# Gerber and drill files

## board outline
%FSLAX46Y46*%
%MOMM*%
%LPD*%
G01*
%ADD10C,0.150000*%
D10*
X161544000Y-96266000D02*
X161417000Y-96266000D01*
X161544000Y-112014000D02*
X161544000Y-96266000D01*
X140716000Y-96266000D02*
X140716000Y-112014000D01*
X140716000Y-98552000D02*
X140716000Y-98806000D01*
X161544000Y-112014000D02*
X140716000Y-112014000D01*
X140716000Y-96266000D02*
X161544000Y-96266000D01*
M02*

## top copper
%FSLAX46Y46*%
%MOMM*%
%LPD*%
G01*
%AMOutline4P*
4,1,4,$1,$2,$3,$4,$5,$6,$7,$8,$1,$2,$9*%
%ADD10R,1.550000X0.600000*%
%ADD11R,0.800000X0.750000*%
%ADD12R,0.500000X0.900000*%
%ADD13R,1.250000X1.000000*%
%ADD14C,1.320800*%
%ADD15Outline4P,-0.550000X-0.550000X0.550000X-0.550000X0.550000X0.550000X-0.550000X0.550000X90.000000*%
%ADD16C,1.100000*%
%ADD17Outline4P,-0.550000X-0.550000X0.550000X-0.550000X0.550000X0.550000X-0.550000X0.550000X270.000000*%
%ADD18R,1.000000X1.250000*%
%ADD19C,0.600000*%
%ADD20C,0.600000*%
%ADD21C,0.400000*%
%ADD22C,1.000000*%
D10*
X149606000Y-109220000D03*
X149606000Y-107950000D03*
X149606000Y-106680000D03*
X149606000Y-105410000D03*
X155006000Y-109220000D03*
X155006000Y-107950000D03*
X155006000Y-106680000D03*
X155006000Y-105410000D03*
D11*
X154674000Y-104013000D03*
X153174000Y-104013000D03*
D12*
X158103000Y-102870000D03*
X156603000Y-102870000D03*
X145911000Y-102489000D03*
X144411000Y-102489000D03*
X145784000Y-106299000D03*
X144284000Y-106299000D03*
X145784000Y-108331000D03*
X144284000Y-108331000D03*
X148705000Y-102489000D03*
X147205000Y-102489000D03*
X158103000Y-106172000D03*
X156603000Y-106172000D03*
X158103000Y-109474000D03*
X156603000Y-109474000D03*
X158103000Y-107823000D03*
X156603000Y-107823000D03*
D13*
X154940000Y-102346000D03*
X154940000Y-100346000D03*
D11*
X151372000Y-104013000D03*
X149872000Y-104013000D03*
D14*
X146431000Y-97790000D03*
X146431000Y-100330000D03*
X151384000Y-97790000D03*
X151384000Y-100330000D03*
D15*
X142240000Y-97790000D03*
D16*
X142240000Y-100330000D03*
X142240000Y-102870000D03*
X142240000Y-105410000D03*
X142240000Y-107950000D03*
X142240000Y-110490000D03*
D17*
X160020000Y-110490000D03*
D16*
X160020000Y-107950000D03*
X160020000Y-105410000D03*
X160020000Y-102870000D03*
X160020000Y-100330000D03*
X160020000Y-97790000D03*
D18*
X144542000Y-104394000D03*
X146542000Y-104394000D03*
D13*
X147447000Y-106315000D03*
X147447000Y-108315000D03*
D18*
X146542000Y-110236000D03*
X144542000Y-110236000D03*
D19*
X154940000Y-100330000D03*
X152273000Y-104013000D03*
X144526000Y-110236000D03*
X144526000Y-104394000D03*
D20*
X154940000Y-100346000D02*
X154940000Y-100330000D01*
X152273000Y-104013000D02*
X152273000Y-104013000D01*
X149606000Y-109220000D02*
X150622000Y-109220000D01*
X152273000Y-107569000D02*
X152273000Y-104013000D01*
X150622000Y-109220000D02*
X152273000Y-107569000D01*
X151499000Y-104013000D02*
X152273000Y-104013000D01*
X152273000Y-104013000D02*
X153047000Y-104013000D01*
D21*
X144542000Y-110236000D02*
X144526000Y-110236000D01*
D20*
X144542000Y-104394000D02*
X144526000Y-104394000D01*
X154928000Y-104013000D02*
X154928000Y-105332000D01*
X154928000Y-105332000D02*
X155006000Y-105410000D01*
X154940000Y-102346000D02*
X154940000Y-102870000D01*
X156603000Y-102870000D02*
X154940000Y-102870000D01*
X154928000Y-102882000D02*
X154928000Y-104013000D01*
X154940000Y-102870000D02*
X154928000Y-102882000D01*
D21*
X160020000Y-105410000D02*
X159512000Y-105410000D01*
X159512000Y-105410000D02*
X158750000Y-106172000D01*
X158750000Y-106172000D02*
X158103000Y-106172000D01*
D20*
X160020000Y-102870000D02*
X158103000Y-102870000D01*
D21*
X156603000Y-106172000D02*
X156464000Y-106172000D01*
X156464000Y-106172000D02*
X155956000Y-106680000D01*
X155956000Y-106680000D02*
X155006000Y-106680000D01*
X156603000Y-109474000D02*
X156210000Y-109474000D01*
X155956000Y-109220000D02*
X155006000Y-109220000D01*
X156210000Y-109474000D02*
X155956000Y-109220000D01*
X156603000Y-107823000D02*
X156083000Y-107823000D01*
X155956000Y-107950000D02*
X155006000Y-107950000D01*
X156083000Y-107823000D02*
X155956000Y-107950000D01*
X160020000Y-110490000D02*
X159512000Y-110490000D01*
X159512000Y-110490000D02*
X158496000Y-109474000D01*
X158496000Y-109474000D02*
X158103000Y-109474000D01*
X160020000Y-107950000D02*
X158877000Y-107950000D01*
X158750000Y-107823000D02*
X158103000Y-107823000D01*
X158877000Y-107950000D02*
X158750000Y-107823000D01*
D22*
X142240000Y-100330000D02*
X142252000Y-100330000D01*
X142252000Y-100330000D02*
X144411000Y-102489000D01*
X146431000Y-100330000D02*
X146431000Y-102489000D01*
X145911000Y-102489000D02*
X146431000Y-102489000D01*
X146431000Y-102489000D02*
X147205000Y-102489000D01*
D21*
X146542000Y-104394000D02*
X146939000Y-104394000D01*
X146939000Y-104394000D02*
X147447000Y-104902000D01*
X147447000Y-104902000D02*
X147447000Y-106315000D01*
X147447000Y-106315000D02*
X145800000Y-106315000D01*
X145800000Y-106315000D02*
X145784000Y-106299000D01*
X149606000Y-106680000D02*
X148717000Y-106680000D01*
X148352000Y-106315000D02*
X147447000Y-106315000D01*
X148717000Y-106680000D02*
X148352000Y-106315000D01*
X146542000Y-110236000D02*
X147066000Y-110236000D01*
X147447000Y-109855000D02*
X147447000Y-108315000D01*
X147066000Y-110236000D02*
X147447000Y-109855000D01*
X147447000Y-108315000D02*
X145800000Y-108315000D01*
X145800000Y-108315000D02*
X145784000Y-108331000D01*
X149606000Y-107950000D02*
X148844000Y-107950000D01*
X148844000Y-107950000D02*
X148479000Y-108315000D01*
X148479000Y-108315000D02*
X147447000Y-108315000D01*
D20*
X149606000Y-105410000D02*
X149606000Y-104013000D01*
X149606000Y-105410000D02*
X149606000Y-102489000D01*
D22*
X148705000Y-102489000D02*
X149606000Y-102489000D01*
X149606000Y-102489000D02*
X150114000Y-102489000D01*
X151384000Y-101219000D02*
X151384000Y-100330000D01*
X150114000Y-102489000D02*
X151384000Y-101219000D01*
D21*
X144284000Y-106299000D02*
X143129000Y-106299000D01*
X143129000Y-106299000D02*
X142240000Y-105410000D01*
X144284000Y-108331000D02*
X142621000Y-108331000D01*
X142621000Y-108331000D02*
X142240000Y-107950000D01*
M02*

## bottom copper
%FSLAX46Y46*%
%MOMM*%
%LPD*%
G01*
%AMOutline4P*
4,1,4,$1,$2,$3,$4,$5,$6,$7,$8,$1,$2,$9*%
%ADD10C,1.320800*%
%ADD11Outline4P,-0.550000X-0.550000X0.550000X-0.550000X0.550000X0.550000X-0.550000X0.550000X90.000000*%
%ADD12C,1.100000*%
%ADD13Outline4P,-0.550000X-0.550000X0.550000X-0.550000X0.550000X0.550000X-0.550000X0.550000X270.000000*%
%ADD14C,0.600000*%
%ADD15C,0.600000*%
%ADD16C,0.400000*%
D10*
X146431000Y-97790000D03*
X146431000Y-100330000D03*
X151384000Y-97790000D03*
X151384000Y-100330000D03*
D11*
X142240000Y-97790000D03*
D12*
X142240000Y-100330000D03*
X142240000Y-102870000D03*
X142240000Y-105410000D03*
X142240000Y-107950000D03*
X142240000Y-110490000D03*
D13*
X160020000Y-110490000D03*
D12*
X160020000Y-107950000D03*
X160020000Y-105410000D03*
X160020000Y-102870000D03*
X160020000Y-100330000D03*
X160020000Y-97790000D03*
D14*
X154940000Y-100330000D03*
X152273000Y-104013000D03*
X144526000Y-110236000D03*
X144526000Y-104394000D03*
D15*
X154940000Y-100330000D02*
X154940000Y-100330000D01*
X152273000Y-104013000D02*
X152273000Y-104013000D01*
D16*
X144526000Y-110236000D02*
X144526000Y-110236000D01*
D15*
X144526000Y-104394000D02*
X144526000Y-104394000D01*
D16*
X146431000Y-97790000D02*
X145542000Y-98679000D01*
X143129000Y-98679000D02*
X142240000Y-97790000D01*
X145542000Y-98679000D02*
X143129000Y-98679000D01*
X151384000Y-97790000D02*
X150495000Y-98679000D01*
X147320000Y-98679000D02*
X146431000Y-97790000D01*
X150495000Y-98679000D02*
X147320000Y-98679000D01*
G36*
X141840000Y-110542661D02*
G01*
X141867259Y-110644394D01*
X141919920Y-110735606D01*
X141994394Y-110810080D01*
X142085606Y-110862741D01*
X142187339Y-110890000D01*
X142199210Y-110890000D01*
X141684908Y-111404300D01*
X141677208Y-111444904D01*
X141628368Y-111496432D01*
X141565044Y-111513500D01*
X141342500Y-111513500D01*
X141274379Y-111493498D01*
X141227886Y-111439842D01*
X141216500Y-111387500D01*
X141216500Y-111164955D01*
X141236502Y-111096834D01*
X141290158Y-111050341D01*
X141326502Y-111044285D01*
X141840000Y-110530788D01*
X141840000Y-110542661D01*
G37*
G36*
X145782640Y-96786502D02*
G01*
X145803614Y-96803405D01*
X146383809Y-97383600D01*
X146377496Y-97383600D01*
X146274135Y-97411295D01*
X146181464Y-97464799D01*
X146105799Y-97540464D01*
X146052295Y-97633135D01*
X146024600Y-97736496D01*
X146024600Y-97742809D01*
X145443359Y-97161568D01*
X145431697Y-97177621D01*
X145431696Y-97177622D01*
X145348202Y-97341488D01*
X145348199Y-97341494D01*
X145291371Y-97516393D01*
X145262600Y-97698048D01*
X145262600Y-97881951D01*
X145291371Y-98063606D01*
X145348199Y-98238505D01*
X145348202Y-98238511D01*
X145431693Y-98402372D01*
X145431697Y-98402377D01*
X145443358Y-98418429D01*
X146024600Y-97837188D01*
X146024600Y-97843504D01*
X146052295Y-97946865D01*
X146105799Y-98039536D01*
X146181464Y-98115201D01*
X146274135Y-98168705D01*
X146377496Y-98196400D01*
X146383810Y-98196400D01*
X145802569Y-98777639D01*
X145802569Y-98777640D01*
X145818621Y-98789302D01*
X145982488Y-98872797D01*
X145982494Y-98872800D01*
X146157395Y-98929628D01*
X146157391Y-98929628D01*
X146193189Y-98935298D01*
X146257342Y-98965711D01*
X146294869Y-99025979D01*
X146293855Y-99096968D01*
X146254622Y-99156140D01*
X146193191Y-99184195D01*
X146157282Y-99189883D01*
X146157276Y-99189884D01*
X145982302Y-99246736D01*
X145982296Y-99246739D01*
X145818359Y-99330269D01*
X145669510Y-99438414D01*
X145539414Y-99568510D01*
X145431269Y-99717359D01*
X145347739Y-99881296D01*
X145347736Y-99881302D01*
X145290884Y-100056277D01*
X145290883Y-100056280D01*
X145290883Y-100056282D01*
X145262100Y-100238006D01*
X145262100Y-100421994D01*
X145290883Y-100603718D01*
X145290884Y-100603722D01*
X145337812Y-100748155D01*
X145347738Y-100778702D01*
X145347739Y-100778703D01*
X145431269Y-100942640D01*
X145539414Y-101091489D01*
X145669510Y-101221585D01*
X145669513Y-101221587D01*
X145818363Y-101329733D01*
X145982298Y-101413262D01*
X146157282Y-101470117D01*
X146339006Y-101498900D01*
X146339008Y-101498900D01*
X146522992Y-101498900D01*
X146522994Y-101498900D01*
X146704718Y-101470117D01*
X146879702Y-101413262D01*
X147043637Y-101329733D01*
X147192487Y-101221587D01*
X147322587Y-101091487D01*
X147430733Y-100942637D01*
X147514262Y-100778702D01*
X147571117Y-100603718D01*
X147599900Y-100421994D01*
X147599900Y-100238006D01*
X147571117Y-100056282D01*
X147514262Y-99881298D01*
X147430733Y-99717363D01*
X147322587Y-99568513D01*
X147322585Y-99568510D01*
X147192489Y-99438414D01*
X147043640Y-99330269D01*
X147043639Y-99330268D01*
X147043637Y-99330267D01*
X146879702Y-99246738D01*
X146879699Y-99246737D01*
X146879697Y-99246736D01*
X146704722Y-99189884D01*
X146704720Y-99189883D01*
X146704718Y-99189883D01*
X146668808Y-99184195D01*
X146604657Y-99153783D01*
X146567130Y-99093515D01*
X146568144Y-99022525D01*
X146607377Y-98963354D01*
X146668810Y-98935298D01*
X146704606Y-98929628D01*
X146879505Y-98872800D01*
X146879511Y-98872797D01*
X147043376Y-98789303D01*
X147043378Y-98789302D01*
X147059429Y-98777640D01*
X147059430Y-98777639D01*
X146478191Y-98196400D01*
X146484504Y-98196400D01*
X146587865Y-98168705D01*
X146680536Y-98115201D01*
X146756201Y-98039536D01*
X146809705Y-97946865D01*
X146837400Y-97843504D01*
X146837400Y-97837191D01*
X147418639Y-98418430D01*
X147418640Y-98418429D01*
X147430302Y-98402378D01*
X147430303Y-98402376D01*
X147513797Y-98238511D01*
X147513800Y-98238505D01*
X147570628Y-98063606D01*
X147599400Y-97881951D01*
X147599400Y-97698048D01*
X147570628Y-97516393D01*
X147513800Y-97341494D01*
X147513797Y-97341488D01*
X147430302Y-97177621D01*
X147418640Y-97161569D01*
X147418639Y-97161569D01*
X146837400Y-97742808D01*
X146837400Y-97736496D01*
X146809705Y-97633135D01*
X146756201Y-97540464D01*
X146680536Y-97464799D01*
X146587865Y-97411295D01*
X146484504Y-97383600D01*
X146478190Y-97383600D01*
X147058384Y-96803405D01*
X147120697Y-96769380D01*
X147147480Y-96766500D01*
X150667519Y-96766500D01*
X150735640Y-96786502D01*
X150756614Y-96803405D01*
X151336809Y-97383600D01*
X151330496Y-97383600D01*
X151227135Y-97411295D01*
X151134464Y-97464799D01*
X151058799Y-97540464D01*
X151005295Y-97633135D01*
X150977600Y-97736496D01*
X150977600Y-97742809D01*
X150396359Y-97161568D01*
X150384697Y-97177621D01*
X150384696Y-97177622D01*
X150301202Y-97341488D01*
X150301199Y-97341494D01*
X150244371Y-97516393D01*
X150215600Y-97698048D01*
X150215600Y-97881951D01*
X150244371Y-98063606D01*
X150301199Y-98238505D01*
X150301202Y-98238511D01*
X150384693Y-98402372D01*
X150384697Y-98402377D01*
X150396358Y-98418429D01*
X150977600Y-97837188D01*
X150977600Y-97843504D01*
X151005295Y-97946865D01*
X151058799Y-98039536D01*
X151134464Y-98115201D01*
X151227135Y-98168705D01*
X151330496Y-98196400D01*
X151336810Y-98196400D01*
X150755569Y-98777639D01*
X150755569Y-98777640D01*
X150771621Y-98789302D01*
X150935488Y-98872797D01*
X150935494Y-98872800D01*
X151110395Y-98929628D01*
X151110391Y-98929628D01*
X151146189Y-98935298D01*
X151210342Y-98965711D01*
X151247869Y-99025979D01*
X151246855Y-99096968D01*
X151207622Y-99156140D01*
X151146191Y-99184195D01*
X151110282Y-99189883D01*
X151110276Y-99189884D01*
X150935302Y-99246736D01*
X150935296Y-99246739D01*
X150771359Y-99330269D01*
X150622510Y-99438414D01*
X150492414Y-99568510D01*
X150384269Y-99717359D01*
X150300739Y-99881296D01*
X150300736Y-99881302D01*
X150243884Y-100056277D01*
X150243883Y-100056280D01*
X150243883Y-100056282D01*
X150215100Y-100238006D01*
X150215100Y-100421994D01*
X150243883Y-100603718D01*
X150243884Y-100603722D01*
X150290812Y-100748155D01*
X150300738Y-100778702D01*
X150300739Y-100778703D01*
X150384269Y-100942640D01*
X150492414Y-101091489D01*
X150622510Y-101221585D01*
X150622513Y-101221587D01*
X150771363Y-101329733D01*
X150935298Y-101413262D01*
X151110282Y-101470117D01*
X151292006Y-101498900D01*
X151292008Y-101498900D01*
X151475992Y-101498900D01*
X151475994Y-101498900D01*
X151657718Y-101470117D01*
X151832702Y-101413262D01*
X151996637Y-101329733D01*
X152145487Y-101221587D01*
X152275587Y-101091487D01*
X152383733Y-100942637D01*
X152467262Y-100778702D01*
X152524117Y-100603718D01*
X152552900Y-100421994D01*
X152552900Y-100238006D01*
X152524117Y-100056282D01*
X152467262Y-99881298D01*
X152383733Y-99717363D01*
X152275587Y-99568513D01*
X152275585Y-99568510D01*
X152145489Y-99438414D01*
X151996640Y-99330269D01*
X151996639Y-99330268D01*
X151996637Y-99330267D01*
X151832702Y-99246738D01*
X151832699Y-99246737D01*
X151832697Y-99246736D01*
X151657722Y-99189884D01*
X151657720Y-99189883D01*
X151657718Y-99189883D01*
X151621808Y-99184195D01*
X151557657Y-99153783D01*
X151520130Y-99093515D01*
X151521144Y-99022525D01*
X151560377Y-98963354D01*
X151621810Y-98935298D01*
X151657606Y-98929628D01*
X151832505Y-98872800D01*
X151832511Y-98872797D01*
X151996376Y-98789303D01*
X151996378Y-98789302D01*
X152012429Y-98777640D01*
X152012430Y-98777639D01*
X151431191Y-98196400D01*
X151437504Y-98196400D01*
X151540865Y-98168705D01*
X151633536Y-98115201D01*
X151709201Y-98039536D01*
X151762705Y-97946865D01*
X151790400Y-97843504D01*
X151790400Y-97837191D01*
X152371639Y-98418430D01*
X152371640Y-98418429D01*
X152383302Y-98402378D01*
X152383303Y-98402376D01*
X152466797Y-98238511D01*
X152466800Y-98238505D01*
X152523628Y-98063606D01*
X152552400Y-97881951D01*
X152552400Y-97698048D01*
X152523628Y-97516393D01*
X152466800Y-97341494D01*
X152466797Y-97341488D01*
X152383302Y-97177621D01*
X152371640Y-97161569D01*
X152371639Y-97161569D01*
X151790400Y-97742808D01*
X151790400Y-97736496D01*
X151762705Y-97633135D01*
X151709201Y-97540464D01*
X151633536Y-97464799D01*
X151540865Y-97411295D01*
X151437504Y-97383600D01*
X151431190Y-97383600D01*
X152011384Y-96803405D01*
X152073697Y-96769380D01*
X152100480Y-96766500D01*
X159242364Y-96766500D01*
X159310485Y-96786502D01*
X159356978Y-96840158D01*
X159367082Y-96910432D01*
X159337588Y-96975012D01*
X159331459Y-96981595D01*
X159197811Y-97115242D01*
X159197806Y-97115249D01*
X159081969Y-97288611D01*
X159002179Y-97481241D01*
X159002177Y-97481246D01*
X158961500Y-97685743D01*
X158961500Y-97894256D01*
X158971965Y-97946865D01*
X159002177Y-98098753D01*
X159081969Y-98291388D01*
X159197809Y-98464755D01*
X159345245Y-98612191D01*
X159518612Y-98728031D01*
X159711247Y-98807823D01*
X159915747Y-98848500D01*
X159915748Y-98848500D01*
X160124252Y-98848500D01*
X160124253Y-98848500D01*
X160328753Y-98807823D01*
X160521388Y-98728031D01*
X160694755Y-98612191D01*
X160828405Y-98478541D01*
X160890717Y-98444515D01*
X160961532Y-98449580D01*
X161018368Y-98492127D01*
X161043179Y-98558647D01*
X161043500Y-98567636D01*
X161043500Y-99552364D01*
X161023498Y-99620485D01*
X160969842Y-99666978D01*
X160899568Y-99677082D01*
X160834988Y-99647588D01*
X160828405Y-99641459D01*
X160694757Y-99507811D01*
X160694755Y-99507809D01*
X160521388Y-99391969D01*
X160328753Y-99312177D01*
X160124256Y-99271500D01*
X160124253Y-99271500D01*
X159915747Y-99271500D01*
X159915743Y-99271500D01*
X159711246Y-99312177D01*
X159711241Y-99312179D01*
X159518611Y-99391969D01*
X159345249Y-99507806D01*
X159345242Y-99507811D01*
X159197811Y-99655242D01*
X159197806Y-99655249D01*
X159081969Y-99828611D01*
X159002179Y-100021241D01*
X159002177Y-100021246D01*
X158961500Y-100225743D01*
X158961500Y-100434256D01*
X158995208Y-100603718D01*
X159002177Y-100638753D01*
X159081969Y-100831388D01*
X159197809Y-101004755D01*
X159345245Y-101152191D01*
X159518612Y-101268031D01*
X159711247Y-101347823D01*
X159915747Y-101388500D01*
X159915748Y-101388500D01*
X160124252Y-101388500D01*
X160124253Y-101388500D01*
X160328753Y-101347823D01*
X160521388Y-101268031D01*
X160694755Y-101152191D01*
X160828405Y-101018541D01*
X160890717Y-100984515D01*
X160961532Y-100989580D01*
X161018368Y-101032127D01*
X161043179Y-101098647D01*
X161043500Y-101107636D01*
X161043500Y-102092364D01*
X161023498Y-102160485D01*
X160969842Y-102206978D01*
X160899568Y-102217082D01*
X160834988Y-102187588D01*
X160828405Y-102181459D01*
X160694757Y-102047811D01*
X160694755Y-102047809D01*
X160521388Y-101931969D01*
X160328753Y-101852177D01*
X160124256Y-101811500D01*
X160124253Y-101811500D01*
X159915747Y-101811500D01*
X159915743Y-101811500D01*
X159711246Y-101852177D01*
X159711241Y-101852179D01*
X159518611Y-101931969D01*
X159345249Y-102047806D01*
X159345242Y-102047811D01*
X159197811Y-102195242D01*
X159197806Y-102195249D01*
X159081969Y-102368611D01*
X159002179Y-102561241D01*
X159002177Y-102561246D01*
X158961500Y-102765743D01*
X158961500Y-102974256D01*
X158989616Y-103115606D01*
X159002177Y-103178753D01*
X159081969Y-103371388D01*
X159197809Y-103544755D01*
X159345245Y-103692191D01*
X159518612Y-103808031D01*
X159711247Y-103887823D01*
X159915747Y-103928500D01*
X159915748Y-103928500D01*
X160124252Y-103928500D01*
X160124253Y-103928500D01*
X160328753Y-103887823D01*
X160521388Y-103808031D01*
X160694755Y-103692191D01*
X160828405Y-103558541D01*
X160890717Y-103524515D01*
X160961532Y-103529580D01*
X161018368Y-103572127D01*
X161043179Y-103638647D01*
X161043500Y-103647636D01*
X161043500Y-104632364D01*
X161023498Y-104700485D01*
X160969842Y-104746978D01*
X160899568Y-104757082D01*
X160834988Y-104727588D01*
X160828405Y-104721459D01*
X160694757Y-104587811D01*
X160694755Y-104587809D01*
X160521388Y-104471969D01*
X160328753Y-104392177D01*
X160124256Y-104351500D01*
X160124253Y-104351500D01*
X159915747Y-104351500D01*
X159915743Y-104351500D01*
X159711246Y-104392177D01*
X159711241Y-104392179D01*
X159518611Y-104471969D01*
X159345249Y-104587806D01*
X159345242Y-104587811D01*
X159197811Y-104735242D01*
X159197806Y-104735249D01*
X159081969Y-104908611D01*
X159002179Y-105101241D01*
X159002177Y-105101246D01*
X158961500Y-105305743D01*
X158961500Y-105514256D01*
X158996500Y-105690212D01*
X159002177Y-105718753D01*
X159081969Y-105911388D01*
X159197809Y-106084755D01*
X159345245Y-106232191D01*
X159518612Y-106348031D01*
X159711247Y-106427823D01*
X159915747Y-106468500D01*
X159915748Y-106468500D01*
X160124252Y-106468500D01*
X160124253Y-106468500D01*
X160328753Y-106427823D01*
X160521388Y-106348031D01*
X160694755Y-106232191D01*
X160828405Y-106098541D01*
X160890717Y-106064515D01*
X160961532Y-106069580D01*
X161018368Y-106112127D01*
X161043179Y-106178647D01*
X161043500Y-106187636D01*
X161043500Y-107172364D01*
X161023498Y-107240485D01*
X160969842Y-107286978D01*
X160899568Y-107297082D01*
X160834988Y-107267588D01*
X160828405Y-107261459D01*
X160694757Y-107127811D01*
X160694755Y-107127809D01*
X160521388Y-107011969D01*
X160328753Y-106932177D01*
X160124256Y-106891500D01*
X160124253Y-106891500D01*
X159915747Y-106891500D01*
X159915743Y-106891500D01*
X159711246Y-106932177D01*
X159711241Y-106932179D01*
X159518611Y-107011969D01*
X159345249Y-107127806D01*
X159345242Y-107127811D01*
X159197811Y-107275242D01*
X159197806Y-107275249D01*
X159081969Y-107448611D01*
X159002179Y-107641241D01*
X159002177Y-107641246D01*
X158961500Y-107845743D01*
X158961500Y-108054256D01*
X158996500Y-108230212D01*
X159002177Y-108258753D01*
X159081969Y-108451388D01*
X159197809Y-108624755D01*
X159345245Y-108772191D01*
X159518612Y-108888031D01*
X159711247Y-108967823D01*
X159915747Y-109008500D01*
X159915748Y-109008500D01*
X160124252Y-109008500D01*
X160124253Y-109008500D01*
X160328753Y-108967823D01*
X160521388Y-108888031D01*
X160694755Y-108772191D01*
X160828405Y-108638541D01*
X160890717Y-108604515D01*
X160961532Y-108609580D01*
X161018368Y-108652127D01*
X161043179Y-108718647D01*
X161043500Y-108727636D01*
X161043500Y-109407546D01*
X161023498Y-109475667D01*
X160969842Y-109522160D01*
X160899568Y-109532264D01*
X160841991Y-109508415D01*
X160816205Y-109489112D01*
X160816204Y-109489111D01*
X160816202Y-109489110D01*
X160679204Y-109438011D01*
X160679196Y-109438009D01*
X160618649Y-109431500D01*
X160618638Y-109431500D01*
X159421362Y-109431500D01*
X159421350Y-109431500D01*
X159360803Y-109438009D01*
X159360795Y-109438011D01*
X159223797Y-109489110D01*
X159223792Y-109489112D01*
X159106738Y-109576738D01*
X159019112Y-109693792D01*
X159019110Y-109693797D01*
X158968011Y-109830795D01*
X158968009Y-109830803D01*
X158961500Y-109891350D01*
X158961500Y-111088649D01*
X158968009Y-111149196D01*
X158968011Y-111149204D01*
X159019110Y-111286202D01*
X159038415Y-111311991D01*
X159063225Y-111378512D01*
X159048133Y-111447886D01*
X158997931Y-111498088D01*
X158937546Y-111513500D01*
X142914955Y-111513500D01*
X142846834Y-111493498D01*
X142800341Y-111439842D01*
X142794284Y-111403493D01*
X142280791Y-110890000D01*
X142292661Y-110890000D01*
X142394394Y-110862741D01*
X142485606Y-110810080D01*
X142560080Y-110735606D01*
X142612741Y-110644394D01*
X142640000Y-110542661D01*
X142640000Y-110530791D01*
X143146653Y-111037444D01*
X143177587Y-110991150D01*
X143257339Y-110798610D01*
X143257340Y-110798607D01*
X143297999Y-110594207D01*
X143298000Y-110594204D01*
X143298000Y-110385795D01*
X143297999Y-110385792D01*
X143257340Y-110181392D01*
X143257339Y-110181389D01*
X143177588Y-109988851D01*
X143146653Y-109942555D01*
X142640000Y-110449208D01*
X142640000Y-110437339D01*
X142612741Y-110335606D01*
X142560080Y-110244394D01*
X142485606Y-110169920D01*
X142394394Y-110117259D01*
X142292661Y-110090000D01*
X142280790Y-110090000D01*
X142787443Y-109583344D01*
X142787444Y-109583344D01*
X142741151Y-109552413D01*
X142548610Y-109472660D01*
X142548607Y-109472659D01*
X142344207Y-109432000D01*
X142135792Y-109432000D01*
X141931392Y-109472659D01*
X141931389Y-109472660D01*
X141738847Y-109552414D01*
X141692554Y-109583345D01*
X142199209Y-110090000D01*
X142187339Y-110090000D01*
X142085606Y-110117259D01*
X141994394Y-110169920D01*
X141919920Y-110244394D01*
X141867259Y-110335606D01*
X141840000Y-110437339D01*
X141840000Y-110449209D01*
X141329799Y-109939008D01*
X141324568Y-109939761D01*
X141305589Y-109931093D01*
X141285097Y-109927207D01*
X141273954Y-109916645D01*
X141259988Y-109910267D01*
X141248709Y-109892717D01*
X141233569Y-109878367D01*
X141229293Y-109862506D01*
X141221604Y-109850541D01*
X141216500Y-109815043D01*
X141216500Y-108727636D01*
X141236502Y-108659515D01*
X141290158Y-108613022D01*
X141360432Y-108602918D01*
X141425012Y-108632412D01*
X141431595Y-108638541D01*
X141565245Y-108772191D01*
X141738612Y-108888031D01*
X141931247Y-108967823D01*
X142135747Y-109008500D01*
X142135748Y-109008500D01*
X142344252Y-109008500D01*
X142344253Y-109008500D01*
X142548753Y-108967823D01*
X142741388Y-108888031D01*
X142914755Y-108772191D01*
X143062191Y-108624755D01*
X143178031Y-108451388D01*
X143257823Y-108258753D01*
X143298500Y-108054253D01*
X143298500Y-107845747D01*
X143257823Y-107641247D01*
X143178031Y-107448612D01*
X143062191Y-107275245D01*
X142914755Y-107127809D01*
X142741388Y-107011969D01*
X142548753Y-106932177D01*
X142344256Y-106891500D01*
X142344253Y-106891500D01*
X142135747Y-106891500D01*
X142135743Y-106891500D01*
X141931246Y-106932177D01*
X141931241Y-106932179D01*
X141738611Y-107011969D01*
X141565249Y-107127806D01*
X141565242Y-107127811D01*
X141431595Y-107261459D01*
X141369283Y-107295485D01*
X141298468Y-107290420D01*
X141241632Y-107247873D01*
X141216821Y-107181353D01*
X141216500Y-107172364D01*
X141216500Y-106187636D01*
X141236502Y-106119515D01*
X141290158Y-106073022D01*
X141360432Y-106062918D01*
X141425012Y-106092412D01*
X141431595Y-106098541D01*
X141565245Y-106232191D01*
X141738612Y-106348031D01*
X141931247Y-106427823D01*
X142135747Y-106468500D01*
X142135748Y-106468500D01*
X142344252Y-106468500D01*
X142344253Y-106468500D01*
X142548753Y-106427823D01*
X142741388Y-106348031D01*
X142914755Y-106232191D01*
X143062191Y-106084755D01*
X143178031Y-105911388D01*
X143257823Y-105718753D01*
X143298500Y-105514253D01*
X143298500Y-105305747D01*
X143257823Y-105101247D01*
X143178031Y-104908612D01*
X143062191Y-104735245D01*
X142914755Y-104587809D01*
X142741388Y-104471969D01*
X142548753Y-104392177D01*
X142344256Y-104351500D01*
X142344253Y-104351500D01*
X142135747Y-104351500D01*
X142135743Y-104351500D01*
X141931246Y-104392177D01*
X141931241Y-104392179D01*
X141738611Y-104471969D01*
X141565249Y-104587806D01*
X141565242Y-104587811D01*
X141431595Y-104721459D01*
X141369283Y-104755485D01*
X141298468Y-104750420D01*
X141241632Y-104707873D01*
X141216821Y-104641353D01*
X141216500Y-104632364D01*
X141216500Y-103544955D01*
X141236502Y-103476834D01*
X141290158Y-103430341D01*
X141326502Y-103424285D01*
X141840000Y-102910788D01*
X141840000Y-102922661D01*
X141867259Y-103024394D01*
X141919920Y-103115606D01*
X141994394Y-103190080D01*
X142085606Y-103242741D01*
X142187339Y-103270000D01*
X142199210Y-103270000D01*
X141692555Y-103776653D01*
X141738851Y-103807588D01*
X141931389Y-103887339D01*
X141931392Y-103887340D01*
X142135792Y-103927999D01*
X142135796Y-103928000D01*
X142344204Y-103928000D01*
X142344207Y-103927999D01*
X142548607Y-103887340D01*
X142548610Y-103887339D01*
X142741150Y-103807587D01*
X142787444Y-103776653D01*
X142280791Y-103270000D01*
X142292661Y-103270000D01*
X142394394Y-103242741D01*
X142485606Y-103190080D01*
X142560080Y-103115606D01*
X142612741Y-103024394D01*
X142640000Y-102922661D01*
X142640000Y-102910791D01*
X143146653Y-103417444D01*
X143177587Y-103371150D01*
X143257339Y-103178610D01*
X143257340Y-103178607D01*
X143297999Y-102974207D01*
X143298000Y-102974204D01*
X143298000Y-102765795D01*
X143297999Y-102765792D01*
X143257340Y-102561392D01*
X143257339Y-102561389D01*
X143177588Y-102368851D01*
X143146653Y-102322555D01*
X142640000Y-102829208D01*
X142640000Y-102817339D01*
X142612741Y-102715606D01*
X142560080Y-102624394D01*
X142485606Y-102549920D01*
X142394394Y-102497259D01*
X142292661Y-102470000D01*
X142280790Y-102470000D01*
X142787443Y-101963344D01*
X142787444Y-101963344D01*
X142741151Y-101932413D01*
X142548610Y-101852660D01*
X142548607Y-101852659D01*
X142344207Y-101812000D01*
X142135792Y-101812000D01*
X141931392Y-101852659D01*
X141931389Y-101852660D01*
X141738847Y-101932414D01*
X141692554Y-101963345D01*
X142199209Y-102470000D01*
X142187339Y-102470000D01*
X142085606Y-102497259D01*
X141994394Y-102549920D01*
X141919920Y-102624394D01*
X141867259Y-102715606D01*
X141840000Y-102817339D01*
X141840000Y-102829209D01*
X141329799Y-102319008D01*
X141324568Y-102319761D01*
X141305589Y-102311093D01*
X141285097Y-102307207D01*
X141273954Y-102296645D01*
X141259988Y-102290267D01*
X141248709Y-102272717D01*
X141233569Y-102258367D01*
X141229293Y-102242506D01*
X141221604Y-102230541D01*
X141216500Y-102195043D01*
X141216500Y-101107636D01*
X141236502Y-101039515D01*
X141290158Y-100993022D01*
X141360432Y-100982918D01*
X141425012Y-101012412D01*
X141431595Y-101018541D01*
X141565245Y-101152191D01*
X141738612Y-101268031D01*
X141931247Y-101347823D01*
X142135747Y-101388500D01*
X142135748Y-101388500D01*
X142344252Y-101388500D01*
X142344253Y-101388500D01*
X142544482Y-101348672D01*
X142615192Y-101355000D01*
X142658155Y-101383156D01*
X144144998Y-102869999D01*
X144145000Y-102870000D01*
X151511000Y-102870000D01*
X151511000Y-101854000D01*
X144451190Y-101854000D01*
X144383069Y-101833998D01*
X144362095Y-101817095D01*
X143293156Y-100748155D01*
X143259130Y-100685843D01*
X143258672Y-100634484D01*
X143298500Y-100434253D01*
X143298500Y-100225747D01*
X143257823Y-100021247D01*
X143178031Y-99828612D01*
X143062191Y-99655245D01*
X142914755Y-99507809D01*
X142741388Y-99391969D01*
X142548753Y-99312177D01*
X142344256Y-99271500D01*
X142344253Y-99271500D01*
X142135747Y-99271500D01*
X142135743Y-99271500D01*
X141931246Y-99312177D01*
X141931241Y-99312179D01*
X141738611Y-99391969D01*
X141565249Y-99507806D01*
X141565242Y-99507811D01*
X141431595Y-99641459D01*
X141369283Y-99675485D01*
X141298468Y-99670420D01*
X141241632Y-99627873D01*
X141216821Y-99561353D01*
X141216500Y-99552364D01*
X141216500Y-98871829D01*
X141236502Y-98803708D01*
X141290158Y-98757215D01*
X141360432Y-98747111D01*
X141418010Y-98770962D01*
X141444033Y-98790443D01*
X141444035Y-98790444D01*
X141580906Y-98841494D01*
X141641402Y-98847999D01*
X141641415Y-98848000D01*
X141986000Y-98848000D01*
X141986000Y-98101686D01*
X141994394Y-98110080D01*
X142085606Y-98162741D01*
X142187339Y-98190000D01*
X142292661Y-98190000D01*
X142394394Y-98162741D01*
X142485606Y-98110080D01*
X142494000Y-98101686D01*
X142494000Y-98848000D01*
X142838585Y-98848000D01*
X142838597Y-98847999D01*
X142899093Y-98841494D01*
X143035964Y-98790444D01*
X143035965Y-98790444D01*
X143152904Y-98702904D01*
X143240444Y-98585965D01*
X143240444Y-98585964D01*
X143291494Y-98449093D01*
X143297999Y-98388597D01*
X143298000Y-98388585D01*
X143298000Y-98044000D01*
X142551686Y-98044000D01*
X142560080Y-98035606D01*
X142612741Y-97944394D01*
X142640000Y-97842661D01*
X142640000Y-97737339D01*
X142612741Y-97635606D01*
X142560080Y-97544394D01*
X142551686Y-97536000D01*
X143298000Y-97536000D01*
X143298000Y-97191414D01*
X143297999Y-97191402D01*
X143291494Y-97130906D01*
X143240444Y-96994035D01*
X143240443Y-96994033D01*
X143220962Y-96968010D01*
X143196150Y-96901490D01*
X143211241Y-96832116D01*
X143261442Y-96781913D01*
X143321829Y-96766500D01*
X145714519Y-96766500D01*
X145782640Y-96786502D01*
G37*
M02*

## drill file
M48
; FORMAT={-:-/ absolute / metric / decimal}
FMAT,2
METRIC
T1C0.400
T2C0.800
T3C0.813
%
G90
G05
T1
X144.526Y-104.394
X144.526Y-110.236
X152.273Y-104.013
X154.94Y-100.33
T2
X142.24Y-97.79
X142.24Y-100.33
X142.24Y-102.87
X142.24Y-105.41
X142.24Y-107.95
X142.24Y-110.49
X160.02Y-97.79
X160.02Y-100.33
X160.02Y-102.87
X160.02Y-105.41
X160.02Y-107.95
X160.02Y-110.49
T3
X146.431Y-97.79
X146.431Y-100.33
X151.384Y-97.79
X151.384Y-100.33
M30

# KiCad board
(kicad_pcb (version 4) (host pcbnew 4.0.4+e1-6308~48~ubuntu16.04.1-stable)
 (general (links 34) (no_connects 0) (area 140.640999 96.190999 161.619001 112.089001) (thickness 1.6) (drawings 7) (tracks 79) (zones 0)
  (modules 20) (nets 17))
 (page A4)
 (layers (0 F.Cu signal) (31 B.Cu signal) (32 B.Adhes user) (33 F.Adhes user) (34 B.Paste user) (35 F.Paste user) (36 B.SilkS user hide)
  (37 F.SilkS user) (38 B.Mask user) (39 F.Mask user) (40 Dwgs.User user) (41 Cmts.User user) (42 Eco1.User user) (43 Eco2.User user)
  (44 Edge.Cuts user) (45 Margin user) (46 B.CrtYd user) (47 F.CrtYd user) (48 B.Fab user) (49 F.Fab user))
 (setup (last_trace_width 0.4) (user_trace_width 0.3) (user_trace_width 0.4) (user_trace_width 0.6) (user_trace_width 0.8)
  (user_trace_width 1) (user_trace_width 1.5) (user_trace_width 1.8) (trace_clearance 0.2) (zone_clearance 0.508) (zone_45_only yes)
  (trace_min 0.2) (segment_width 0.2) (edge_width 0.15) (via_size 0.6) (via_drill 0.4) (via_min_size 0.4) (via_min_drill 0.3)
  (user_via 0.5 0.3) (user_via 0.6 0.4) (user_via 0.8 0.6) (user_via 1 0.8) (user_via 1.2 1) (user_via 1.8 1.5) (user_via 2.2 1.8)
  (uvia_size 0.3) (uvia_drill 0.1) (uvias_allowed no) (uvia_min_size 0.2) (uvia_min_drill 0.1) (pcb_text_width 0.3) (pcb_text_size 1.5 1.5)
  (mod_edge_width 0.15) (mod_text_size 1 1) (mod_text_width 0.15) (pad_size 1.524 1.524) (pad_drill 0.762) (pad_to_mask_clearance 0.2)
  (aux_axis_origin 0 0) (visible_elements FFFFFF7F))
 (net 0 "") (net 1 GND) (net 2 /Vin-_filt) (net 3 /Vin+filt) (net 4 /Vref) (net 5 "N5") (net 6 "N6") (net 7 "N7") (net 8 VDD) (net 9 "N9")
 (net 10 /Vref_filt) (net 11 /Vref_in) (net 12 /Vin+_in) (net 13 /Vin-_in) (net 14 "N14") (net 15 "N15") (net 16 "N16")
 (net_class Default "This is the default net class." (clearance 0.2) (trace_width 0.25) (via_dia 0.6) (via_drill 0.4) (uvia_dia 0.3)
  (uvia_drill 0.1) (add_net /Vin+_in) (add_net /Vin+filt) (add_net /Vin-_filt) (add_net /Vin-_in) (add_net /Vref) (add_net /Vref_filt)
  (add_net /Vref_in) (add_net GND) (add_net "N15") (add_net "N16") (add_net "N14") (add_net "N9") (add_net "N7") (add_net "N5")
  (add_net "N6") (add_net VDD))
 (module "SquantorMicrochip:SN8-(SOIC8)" (layer F.Cu) (at 152.273 107.315)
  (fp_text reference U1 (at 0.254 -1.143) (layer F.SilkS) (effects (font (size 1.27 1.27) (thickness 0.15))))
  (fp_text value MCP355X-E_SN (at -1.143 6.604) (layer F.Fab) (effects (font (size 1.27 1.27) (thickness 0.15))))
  (pad 4 smd rect (at -2.667 1.905 270) (size 0.6 1.55) (layers F.Cu F.Paste F.Mask) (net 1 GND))
  (pad 3 smd rect (at -2.667 0.635 270) (size 0.6 1.55) (layers F.Cu F.Paste F.Mask) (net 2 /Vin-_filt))
  (pad 2 smd rect (at -2.667 -0.635 270) (size 0.6 1.55) (layers F.Cu F.Paste F.Mask) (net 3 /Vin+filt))
  (pad 1 smd rect (at -2.667 -1.905 270) (size 0.6 1.55) (layers F.Cu F.Paste F.Mask) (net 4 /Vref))
  (pad 5 smd rect (at 2.733 1.905 270) (size 0.6 1.55) (layers F.Cu F.Paste F.Mask) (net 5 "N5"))
  (pad 6 smd rect (at 2.733 0.635 270) (size 0.6 1.55) (layers F.Cu F.Paste F.Mask) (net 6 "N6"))
  (pad 7 smd rect (at 2.733 -0.635 270) (size 0.6 1.55) (layers F.Cu F.Paste F.Mask) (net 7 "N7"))
  (pad 8 smd rect (at 2.733 -1.905 270) (size 0.6 1.55) (layers F.Cu F.Paste F.Mask) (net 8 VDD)))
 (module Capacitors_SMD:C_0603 (layer F.Cu) (at 153.924 104.013 180)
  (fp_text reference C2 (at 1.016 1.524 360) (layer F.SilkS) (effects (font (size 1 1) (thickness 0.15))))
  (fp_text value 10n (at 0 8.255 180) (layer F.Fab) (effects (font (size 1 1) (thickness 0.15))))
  (pad 1 smd rect (at -0.75 0 180) (size 0.8 0.75) (layers F.Cu F.Paste F.Mask) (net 8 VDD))
  (pad 2 smd rect (at 0.75 0 180) (size 0.8 0.75) (layers F.Cu F.Paste F.Mask) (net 1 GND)))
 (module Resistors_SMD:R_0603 (layer F.Cu) (at 157.353 102.87 180)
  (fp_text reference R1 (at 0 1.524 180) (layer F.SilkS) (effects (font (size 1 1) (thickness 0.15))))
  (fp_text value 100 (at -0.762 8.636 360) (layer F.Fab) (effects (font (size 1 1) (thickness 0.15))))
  (pad 1 smd rect (at -0.75 0 180) (size 0.5 0.9) (layers F.Cu F.Paste F.Mask) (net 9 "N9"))
  (pad 2 smd rect (at 0.75 0 180) (size 0.5 0.9) (layers F.Cu F.Paste F.Mask) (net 8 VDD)))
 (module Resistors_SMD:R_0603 (layer F.Cu) (at 145.161 102.489 180)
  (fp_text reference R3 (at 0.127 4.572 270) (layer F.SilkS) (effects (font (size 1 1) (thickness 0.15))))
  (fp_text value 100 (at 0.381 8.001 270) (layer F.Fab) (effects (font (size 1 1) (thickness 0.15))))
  (pad 1 smd rect (at -0.75 0 180) (size 0.5 0.9) (layers F.Cu F.Paste F.Mask) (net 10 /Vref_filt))
  (pad 2 smd rect (at 0.75 0 180) (size 0.5 0.9) (layers F.Cu F.Paste F.Mask) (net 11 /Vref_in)))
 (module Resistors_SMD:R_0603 (layer F.Cu) (at 145.034 106.299 180)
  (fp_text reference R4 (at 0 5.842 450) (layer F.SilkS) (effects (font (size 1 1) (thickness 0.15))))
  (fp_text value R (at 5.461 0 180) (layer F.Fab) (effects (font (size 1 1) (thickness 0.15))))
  (pad 1 smd rect (at -0.75 0 180) (size 0.5 0.9) (layers F.Cu F.Paste F.Mask) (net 3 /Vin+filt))
  (pad 2 smd rect (at 0.75 0 180) (size 0.5 0.9) (layers F.Cu F.Paste F.Mask) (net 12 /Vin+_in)))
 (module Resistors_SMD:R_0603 (layer F.Cu) (at 145.034 108.331 180)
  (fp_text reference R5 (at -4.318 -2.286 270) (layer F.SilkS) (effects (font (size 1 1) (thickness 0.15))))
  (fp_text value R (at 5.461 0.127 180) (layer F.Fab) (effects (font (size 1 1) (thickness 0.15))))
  (pad 1 smd rect (at -0.75 0 180) (size 0.5 0.9) (layers F.Cu F.Paste F.Mask) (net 2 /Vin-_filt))
  (pad 2 smd rect (at 0.75 0 180) (size 0.5 0.9) (layers F.Cu F.Paste F.Mask) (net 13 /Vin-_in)))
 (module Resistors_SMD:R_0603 (layer F.Cu) (at 147.955 102.489 180)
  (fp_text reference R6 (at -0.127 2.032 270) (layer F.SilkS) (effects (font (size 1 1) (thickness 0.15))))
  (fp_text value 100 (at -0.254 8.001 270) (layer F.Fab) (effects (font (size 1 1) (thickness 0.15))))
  (pad 1 smd rect (at -0.75 0 180) (size 0.5 0.9) (layers F.Cu F.Paste F.Mask) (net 4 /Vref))
  (pad 2 smd rect (at 0.75 0 180) (size 0.5 0.9) (layers F.Cu F.Paste F.Mask) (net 10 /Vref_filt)))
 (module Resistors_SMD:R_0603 (layer F.Cu) (at 157.353 106.172 180)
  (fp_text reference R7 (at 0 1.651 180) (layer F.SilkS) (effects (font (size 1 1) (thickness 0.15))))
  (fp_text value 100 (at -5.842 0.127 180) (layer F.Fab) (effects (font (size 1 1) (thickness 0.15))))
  (pad 1 smd rect (at -0.75 0 180) (size 0.5 0.9) (layers F.Cu F.Paste F.Mask) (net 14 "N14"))
  (pad 2 smd rect (at 0.75 0 180) (size 0.5 0.9) (layers F.Cu F.Paste F.Mask) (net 7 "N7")))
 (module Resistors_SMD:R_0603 (layer F.Cu) (at 157.353 109.474 180)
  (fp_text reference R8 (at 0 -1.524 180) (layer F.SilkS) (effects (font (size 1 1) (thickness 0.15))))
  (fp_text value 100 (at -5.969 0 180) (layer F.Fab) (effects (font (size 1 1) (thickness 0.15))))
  (pad 1 smd rect (at -0.75 0 180) (size 0.5 0.9) (layers F.Cu F.Paste F.Mask) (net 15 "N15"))
  (pad 2 smd rect (at 0.75 0 180) (size 0.5 0.9) (layers F.Cu F.Paste F.Mask) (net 5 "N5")))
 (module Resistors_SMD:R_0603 (layer F.Cu) (at 157.353 107.823 180)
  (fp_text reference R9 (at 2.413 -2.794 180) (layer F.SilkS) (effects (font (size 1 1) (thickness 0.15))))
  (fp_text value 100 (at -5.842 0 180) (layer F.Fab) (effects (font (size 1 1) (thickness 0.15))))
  (pad 1 smd rect (at -0.75 0 180) (size 0.5 0.9) (layers F.Cu F.Paste F.Mask) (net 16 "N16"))
  (pad 2 smd rect (at 0.75 0 180) (size 0.5 0.9) (layers F.Cu F.Paste F.Mask) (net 6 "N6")))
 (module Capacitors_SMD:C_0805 (layer F.Cu) (at 154.94 101.346 90)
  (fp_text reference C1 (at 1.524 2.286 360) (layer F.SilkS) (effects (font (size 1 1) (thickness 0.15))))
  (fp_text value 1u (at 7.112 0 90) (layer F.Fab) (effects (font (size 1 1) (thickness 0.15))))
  (pad 1 smd rect (at -1 0 90) (size 1 1.25) (layers F.Cu F.Paste F.Mask) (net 8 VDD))
  (pad 2 smd rect (at 1 0 90) (size 1 1.25) (layers F.Cu F.Paste F.Mask) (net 1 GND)))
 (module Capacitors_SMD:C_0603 (layer F.Cu) (at 150.622 104.013 180)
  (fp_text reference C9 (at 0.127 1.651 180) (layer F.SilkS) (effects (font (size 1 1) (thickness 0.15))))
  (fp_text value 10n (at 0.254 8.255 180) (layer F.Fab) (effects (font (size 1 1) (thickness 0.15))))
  (pad 1 smd rect (at -0.75 0 180) (size 0.8 0.75) (layers F.Cu F.Paste F.Mask) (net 1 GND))
  (pad 2 smd rect (at 0.75 0 180) (size 0.8 0.75) (layers F.Cu F.Paste F.Mask) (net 4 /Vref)))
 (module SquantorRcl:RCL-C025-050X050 (layer F.Cu) (at 146.431 99.06 270)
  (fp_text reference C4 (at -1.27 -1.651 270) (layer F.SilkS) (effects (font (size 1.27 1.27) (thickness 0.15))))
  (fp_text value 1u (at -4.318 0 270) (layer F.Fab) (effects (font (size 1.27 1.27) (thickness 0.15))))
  (pad 1 thru_hole circle (at -1.27 0 270) (size 1.3208 1.3208) (drill 0.8128) (layers *.Cu *.Mask F.Paste F.SilkS) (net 1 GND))
  (pad 2 thru_hole circle (at 1.27 0 270) (size 1.3208 1.3208) (drill 0.8128) (layers *.Cu *.Mask F.Paste F.SilkS) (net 10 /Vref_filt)))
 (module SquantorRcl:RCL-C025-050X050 (layer F.Cu) (at 151.384 99.06 270)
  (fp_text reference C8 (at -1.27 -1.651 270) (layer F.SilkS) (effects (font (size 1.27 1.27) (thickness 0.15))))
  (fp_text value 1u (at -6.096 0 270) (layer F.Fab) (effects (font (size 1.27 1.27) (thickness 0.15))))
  (pad 1 thru_hole circle (at -1.27 0 270) (size 1.3208 1.3208) (drill 0.8128) (layers *.Cu *.Mask F.Paste F.SilkS) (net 1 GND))
  (pad 2 thru_hole circle (at 1.27 0 270) (size 1.3208 1.3208) (drill 0.8128) (layers *.Cu *.Mask F.Paste F.SilkS) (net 4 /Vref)))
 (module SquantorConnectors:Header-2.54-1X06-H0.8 (layer B.Cu) (at 142.24 104.14 270)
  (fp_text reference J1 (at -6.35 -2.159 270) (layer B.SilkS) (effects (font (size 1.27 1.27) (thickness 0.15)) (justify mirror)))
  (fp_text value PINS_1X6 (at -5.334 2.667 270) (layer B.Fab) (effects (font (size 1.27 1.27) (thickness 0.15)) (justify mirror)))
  (pad 1 thru_hole trapezoid (at -6.35 0 90) (size 1.1 1.1) (drill 0.8) (layers *.Cu *.Mask) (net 1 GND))
  (pad 2 thru_hole circle (at -3.81 0 90) (size 1.1 1.1) (drill 0.8) (layers *.Cu *.Mask) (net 11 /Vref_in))
  (pad 3 thru_hole circle (at -1.27 0 90) (size 1.1 1.1) (drill 0.8) (layers *.Cu *.Mask) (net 1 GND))
  (pad 4 thru_hole circle (at 1.27 0 90) (size 1.1 1.1) (drill 0.8) (layers *.Cu *.Mask) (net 12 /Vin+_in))
  (pad 5 thru_hole circle (at 3.81 0 90) (size 1.1 1.1) (drill 0.8) (layers *.Cu *.Mask) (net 13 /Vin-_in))
  (pad 6 thru_hole circle (at 6.35 0 90) (size 1.1 1.1) (drill 0.8) (layers *.Cu *.Mask) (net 1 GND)))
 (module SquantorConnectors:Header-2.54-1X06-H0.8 (layer B.Cu) (at 160.02 104.14 90)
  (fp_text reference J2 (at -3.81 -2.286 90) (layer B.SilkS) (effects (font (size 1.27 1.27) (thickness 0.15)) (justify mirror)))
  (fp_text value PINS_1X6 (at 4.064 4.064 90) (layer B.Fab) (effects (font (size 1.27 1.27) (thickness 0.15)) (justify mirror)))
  (pad 1 thru_hole trapezoid (at -6.35 0 270) (size 1.1 1.1) (drill 0.8) (layers *.Cu *.Mask) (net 15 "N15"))
  (pad 2 thru_hole circle (at -3.81 0 270) (size 1.1 1.1) (drill 0.8) (layers *.Cu *.Mask) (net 16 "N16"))
  (pad 3 thru_hole circle (at -1.27 0 270) (size 1.1 1.1) (drill 0.8) (layers *.Cu *.Mask) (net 14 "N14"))
  (pad 4 thru_hole circle (at 1.27 0 270) (size 1.1 1.1) (drill 0.8) (layers *.Cu *.Mask) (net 9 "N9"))
  (pad 5 thru_hole circle (at 3.81 0 270) (size 1.1 1.1) (drill 0.8) (layers *.Cu *.Mask))
  (pad 6 thru_hole circle (at 6.35 0 270) (size 1.1 1.1) (drill 0.8) (layers *.Cu *.Mask)))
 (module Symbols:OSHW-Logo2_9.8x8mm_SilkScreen (layer B.Cu) (at 151.638 105.537 180)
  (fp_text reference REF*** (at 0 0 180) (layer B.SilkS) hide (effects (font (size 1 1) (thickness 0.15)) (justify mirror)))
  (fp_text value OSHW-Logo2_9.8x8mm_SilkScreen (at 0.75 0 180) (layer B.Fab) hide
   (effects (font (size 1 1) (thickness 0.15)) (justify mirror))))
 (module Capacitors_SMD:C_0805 (layer F.Cu) (at 145.542 104.394)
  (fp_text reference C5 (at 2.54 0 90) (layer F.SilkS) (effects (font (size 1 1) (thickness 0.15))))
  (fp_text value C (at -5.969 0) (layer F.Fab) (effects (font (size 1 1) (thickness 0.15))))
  (pad 1 smd rect (at -1 0) (size 1 1.25) (layers F.Cu F.Paste F.Mask) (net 1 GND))
  (pad 2 smd rect (at 1 0) (size 1 1.25) (layers F.Cu F.Paste F.Mask) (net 3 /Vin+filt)))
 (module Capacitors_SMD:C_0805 (layer F.Cu) (at 147.447 107.315 270)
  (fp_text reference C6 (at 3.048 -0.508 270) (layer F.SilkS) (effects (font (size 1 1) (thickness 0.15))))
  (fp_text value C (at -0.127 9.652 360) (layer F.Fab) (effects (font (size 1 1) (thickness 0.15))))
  (pad 1 smd rect (at -1 0 270) (size 1 1.25) (layers F.Cu F.Paste F.Mask) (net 3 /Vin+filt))
  (pad 2 smd rect (at 1 0 270) (size 1 1.25) (layers F.Cu F.Paste F.Mask) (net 2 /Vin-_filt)))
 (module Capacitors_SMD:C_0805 (layer F.Cu) (at 145.542 110.236 180)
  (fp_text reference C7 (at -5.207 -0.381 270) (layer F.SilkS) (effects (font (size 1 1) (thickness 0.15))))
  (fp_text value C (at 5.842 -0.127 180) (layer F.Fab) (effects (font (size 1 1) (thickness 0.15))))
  (pad 1 smd rect (at -1 0 180) (size 1 1.25) (layers F.Cu F.Paste F.Mask) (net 2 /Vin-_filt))
  (pad 2 smd rect (at 1 0 180) (size 1 1.25) (layers F.Cu F.Paste F.Mask) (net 1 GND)))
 (gr_line (start 161.544 96.266) (end 161.417 96.266) (angle 90) (layer Edge.Cuts) (width 0.15))
 (gr_line (start 161.544 112.014) (end 161.544 96.266) (angle 90) (layer Edge.Cuts) (width 0.15))
 (gr_line (start 140.716 96.266) (end 140.716 112.014) (angle 90) (layer Edge.Cuts) (width 0.15))
 (gr_line (start 140.716 98.552) (end 140.716 98.806) (angle 90) (layer Edge.Cuts) (width 0.15))
 (gr_line (start 161.544 112.014) (end 140.716 112.014) (angle 90) (layer Edge.Cuts) (width 0.15))
 (gr_line (start 140.716 96.266) (end 161.544 96.266) (angle 90) (layer Edge.Cuts) (width 0.15))
 (segment (start 154.94 100.346) (end 154.94 100.33) (width 0.6) (layer F.Cu) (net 1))
 (segment (start 154.94 100.33) (end 154.94 100.33) (width 0.6) (layer B.Cu) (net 1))
 (via (at 154.94 100.33) (size 0.6) (drill 0.4) (layers F.Cu B.Cu) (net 1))
 (segment (start 152.273 104.013) (end 152.273 104.013) (width 0.6) (layer F.Cu) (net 1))
 (segment (start 152.273 104.013) (end 152.273 104.013) (width 0.6) (layer B.Cu) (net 1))
 (via (at 152.273 104.013) (size 0.6) (drill 0.4) (layers F.Cu B.Cu) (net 1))
 (segment (start 149.606 109.22) (end 150.622 109.22) (width 0.6) (layer F.Cu) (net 1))
 (segment (start 152.273 107.569) (end 152.273 104.013) (width 0.6) (layer F.Cu) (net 1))
 (segment (start 150.622 109.22) (end 152.273 107.569) (width 0.6) (layer F.Cu) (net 1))
 (segment (start 151.499 104.013) (end 152.273 104.013) (width 0.6) (layer F.Cu) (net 1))
 (segment (start 152.273 104.013) (end 153.047 104.013) (width 0.6) (layer F.Cu) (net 1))
 (segment (start 144.542 110.236) (end 144.526 110.236) (width 0.4) (layer F.Cu) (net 1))
 (segment (start 144.526 110.236) (end 144.526 110.236) (width 0.4) (layer B.Cu) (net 1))
 (via (at 144.526 110.236) (size 0.6) (drill 0.4) (layers F.Cu B.Cu) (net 1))
 (segment (start 144.542 104.394) (end 144.526 104.394) (width 0.6) (layer F.Cu) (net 1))
 (segment (start 144.526 104.394) (end 144.526 104.394) (width 0.6) (layer B.Cu) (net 1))
 (via (at 144.526 104.394) (size 0.6) (drill 0.4) (layers F.Cu B.Cu) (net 1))
 (segment (start 146.431 97.79) (end 145.542 98.679) (width 0.4) (layer B.Cu) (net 1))
 (segment (start 143.129 98.679) (end 142.24 97.79) (width 0.4) (layer B.Cu) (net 1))
 (segment (start 145.542 98.679) (end 143.129 98.679) (width 0.4) (layer B.Cu) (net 1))
 (segment (start 151.384 97.79) (end 150.495 98.679) (width 0.4) (layer B.Cu) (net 1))
 (segment (start 147.32 98.679) (end 146.431 97.79) (width 0.4) (layer B.Cu) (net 1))
 (segment (start 150.495 98.679) (end 147.32 98.679) (width 0.4) (layer B.Cu) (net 1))
 (segment (start 154.928 104.013) (end 154.928 105.332) (width 0.6) (layer F.Cu) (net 8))
 (segment (start 154.928 105.332) (end 155.006 105.41) (width 0.6) (layer F.Cu) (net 8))
 (segment (start 154.94 102.346) (end 154.94 102.87) (width 0.6) (layer F.Cu) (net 8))
 (segment (start 156.603 102.87) (end 154.94 102.87) (width 0.6) (layer F.Cu) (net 8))
 (segment (start 154.928 102.882) (end 154.928 104.013) (width 0.6) (layer F.Cu) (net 8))
 (segment (start 154.94 102.87) (end 154.928 102.882) (width 0.6) (layer F.Cu) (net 8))
 (segment (start 160.02 105.41) (end 159.512 105.41) (width 0.4) (layer F.Cu) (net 14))
 (segment (start 159.512 105.41) (end 158.75 106.172) (width 0.4) (layer F.Cu) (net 14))
 (segment (start 158.75 106.172) (end 158.103 106.172) (width 0.4) (layer F.Cu) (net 14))
 (segment (start 160.02 102.87) (end 158.103 102.87) (width 0.6) (layer F.Cu) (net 9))
 (segment (start 156.603 106.172) (end 156.464 106.172) (width 0.4) (layer F.Cu) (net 7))
 (segment (start 156.464 106.172) (end 155.956 106.68) (width 0.4) (layer F.Cu) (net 7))
 (segment (start 155.956 106.68) (end 155.006 106.68) (width 0.4) (layer F.Cu) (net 7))
 (segment (start 156.603 109.474) (end 156.21 109.474) (width 0.4) (layer F.Cu) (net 5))
 (segment (start 155.956 109.22) (end 155.006 109.22) (width 0.4) (layer F.Cu) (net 5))
 (segment (start 156.21 109.474) (end 155.956 109.22) (width 0.4) (layer F.Cu) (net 5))
 (segment (start 156.603 107.823) (end 156.083 107.823) (width 0.4) (layer F.Cu) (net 6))
 (segment (start 155.956 107.95) (end 155.006 107.95) (width 0.4) (layer F.Cu) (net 6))
 (segment (start 156.083 107.823) (end 155.956 107.95) (width 0.4) (layer F.Cu) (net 6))
 (segment (start 160.02 110.49) (end 159.512 110.49) (width 0.4) (layer F.Cu) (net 15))
 (segment (start 159.512 110.49) (end 158.496 109.474) (width 0.4) (layer F.Cu) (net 15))
 (segment (start 158.496 109.474) (end 158.103 109.474) (width 0.4) (layer F.Cu) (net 15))
 (segment (start 160.02 107.95) (end 158.877 107.95) (width 0.4) (layer F.Cu) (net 16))
 (segment (start 158.75 107.823) (end 158.103 107.823) (width 0.4) (layer F.Cu) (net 16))
 (segment (start 158.877 107.95) (end 158.75 107.823) (width 0.4) (layer F.Cu) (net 16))
 (segment (start 142.24 100.33) (end 142.252 100.33) (width 1) (layer F.Cu) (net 11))
 (segment (start 142.252 100.33) (end 144.411 102.489) (width 1) (layer F.Cu) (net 11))
 (segment (start 146.431 100.33) (end 146.431 102.489) (width 1) (layer F.Cu) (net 10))
 (segment (start 145.911 102.489) (end 146.431 102.489) (width 1) (layer F.Cu) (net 10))
 (segment (start 146.431 102.489) (end 147.205 102.489) (width 1) (layer F.Cu) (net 10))
 (segment (start 146.542 104.394) (end 146.939 104.394) (width 0.4) (layer F.Cu) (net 3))
 (segment (start 146.939 104.394) (end 147.447 104.902) (width 0.4) (layer F.Cu) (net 3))
 (segment (start 147.447 104.902) (end 147.447 106.315) (width 0.4) (layer F.Cu) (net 3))
 (segment (start 147.447 106.315) (end 145.8 106.315) (width 0.4) (layer F.Cu) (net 3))
 (segment (start 145.8 106.315) (end 145.784 106.299) (width 0.4) (layer F.Cu) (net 3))
 (segment (start 149.606 106.68) (end 148.717 106.68) (width 0.4) (layer F.Cu) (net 3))
 (segment (start 148.352 106.315) (end 147.447 106.315) (width 0.4) (layer F.Cu) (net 3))
 (segment (start 148.717 106.68) (end 148.352 106.315) (width 0.4) (layer F.Cu) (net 3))
 (segment (start 146.542 110.236) (end 147.066 110.236) (width 0.4) (layer F.Cu) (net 2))
 (segment (start 147.447 109.855) (end 147.447 108.315) (width 0.4) (layer F.Cu) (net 2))
 (segment (start 147.066 110.236) (end 147.447 109.855) (width 0.4) (layer F.Cu) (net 2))
 (segment (start 147.447 108.315) (end 145.8 108.315) (width 0.4) (layer F.Cu) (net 2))
 (segment (start 145.8 108.315) (end 145.784 108.331) (width 0.4) (layer F.Cu) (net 2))
 (segment (start 149.606 107.95) (end 148.844 107.95) (width 0.4) (layer F.Cu) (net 2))
 (segment (start 148.844 107.95) (end 148.479 108.315) (width 0.4) (layer F.Cu) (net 2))
 (segment (start 148.479 108.315) (end 147.447 108.315) (width 0.4) (layer F.Cu) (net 2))
 (segment (start 149.606 105.41) (end 149.606 104.013) (width 0.6) (layer F.Cu) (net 4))
 (segment (start 149.606 105.41) (end 149.606 102.489) (width 0.6) (layer F.Cu) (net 4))
 (segment (start 148.705 102.489) (end 149.606 102.489) (width 1) (layer F.Cu) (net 4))
 (segment (start 149.606 102.489) (end 150.114 102.489) (width 1) (layer F.Cu) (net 4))
 (segment (start 151.384 101.219) (end 151.384 100.33) (width 1) (layer F.Cu) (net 4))
 (segment (start 150.114 102.489) (end 151.384 101.219) (width 1) (layer F.Cu) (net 4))
 (segment (start 144.284 106.299) (end 143.129 106.299) (width 0.4) (layer F.Cu) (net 12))
 (segment (start 143.129 106.299) (end 142.24 105.41) (width 0.4) (layer F.Cu) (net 12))
 (segment (start 144.284 108.331) (end 142.621 108.331) (width 0.4) (layer F.Cu) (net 13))
 (segment (start 142.621 108.331) (end 142.24 107.95) (width 0.4) (layer F.Cu) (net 13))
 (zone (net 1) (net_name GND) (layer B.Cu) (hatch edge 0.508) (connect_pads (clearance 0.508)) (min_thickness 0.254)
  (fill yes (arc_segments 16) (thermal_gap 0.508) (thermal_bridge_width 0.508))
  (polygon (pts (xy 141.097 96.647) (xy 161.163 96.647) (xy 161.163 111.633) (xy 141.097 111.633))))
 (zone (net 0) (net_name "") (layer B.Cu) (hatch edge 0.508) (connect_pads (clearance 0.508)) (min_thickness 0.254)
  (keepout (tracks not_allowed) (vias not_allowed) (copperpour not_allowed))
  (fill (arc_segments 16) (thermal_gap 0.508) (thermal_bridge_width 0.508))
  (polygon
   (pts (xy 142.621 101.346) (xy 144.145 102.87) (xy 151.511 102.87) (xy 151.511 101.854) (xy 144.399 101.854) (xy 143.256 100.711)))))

